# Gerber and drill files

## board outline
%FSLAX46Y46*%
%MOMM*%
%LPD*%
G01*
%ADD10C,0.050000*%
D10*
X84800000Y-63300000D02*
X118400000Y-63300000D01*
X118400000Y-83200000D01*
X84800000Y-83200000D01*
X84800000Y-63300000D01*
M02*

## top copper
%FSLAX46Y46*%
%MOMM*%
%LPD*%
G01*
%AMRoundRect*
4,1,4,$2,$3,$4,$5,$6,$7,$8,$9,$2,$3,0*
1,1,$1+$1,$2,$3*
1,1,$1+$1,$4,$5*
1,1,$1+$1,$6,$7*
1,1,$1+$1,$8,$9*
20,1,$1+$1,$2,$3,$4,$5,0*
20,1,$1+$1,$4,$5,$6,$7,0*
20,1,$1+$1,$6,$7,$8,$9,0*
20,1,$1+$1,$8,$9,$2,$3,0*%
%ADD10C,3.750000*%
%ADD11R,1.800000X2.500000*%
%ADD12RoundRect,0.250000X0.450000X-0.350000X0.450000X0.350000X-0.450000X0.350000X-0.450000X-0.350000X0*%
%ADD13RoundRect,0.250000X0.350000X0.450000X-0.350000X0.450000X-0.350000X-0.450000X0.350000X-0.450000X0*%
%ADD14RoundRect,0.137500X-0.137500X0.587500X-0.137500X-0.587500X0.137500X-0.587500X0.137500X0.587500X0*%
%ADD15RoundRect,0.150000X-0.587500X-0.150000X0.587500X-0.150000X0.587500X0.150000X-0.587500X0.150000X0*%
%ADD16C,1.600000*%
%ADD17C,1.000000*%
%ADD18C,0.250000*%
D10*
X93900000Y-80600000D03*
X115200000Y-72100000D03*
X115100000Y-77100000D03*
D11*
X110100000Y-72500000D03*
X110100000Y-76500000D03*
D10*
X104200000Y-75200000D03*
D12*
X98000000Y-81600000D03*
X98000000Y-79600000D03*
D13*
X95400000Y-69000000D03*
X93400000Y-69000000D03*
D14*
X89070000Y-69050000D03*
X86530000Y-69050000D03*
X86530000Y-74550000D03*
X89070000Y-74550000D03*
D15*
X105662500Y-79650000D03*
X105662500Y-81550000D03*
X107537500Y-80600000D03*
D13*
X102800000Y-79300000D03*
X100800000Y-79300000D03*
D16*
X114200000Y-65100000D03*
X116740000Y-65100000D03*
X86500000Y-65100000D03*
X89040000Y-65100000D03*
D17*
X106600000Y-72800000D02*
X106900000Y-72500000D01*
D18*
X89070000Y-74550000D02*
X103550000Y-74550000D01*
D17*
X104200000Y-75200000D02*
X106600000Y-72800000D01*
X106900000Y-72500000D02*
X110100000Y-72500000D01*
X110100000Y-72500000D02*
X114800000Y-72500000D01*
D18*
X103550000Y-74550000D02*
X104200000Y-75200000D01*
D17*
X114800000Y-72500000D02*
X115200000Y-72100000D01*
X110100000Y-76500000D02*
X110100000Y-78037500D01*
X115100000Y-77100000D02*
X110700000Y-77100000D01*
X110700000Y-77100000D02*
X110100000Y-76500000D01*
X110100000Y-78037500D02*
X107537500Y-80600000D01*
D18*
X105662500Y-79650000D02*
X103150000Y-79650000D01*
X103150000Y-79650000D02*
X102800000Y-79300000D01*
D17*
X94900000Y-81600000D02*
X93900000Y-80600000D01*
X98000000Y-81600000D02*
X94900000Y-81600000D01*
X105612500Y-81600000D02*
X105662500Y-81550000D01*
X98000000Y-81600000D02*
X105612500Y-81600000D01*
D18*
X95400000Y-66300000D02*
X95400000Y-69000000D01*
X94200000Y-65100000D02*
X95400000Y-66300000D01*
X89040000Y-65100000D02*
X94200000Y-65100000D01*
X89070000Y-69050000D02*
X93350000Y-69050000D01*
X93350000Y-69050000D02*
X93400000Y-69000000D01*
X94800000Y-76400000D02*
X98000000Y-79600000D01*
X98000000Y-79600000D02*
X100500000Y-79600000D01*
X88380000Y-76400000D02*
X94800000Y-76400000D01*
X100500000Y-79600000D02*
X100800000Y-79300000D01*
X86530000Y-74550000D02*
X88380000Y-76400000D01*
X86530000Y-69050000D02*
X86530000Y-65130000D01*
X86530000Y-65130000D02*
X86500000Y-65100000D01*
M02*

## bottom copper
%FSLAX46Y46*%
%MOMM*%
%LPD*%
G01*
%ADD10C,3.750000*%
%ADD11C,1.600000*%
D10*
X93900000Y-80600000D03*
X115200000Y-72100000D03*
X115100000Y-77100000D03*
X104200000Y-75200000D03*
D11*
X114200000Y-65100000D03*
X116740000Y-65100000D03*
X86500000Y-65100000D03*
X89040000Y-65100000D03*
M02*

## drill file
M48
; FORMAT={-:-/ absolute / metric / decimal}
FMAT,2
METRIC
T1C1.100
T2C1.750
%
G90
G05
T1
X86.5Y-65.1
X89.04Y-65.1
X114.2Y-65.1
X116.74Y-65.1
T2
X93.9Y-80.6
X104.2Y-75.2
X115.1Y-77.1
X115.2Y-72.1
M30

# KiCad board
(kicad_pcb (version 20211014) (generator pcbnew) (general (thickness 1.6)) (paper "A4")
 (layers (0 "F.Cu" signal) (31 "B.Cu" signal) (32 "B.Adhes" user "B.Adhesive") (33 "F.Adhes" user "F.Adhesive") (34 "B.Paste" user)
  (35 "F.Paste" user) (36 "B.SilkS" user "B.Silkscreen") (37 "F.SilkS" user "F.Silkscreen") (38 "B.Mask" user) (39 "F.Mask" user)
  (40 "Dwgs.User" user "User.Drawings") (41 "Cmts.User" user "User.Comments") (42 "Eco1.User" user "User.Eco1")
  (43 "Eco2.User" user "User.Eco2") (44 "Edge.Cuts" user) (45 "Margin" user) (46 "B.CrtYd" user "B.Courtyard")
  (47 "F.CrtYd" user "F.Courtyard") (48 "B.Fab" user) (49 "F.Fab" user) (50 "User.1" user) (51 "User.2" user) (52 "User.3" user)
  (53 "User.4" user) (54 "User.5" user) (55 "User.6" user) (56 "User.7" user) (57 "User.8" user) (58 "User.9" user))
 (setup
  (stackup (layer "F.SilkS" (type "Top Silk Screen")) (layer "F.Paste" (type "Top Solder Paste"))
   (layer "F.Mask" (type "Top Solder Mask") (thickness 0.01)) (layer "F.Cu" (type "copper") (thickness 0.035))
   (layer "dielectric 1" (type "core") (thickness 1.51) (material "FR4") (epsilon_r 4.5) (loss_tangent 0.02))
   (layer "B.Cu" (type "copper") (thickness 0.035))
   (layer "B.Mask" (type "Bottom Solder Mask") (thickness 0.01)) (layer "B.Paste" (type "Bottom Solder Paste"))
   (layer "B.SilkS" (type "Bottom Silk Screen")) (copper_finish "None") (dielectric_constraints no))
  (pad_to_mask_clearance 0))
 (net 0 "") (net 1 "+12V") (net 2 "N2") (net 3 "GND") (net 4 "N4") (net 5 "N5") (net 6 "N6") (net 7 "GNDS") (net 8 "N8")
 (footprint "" (layer "F.Cu") (at 93.9 80.6)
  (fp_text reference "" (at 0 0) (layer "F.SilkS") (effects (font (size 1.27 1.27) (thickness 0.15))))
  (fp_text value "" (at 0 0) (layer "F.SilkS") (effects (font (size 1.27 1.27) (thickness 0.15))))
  (pad "3" thru_hole circle (at 0 0 270) (size 3.75 3.75) (drill 1.75) (layers *.Cu *.Mask "B.SilkS")))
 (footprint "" (layer "F.Cu") (at 115.2 72.1)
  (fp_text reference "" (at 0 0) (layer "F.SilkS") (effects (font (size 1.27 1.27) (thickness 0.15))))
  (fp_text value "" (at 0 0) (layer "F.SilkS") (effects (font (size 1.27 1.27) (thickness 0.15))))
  (pad "3" thru_hole circle (at 0 0 270) (size 3.75 3.75) (drill 1.75) (layers *.Cu *.Mask "B.SilkS")))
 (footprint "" (layer "F.Cu") (at 115.1 77.1)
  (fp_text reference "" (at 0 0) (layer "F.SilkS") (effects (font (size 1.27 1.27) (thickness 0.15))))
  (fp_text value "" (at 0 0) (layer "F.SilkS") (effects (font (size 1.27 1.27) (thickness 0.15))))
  (pad "3" thru_hole circle (at 0 0 270) (size 3.75 3.75) (drill 1.75) (layers *.Cu *.Mask "B.SilkS")))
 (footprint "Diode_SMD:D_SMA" (layer "F.Cu") (at 110.1 74.5 -90)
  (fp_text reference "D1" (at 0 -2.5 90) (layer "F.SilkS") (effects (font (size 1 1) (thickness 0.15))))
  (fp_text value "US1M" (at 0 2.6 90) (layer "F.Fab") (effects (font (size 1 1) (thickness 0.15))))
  (pad "1" smd rect (at -2 0 270) (size 2.5 1.8) (layers "F.Cu" "F.Paste" "F.Mask") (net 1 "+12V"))
  (pad "2" smd rect (at 2 0 270) (size 2.5 1.8) (layers "F.Cu" "F.Paste" "F.Mask") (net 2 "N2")))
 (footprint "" (layer "F.Cu") (at 104.2 75.2)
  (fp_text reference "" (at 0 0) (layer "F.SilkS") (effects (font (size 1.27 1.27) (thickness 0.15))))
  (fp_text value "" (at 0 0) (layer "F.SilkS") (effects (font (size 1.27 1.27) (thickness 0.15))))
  (pad "3" thru_hole circle (at 0 0 270) (size 3.75 3.75) (drill 1.75) (layers *.Cu *.Mask "B.SilkS")))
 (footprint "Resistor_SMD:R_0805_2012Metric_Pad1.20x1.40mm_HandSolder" (layer "F.Cu") (at 98 80.6 90)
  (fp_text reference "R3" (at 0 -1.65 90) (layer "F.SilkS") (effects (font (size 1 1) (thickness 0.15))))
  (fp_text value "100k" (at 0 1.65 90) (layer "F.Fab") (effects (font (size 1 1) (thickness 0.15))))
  (pad "1" smd roundrect (at -1 0 90) (size 1.2 1.4) (layers "F.Cu" "F.Paste" "F.Mask") (roundrect_rratio 0.2083333333) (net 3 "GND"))
  (pad "2" smd roundrect (at 1 0 90) (size 1.2 1.4) (layers "F.Cu" "F.Paste" "F.Mask") (roundrect_rratio 0.2083333333) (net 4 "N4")))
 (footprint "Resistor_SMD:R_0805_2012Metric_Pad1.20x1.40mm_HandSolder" (layer "F.Cu") (at 94.4 69 180)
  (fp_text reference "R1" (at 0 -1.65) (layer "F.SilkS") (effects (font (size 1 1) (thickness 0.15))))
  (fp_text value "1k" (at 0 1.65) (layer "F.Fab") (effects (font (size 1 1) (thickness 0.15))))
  (pad "1" smd roundrect (at -1 0 180) (size 1.2 1.4) (layers "F.Cu" "F.Paste" "F.Mask") (roundrect_rratio 0.2083333333) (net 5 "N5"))
  (pad "2" smd roundrect (at 1 0 180) (size 1.2 1.4) (layers "F.Cu" "F.Paste" "F.Mask") (roundrect_rratio 0.2083333333) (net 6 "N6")))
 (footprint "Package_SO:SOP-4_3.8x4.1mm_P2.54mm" (layer "F.Cu") (at 87.8 71.8 -90)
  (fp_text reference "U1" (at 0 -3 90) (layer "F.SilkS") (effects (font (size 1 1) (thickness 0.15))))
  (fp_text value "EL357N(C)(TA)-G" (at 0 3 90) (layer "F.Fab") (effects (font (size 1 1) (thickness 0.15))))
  (pad "1" smd roundrect (at -2.75 -1.27 270) (size 1.45 0.55) (layers "F.Cu" "F.Paste" "F.Mask") (roundrect_rratio 0.25) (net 6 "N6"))
  (pad "2" smd roundrect (at -2.75 1.27 270) (size 1.45 0.55) (layers "F.Cu" "F.Paste" "F.Mask") (roundrect_rratio 0.25) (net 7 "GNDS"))
  (pad "3" smd roundrect (at 2.75 1.27 270) (size 1.45 0.55) (layers "F.Cu" "F.Paste" "F.Mask") (roundrect_rratio 0.25) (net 4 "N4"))
  (pad "4" smd roundrect (at 2.75 -1.27 270) (size 1.45 0.55) (layers "F.Cu" "F.Paste" "F.Mask") (roundrect_rratio 0.25) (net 1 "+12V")))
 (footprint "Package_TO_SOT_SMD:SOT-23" (layer "F.Cu") (at 106.6 80.6)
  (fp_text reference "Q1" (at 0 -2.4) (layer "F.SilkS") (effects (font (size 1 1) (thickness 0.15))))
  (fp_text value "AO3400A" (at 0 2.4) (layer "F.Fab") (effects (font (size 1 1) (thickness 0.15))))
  (pad "1" smd roundrect (at -0.9375 -0.95) (size 1.475 0.6) (layers "F.Cu" "F.Paste" "F.Mask") (roundrect_rratio 0.25) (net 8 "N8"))
  (pad "2" smd roundrect (at -0.9375 0.95) (size 1.475 0.6) (layers "F.Cu" "F.Paste" "F.Mask") (roundrect_rratio 0.25) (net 3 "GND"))
  (pad "3" smd roundrect (at 0.9375 0) (size 1.475 0.6) (layers "F.Cu" "F.Paste" "F.Mask") (roundrect_rratio 0.25) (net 2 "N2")))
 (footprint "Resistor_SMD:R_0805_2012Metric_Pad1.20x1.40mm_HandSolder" (layer "F.Cu") (at 101.8 79.3 180)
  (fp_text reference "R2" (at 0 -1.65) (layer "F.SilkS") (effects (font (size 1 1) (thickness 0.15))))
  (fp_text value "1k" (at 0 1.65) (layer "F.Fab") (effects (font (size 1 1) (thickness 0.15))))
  (pad "1" smd roundrect (at -1 0 180) (size 1.2 1.4) (layers "F.Cu" "F.Paste" "F.Mask") (roundrect_rratio 0.2083333333) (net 8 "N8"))
  (pad "2" smd roundrect (at 1 0 180) (size 1.2 1.4) (layers "F.Cu" "F.Paste" "F.Mask") (roundrect_rratio 0.2083333333) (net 4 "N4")))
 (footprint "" (layer "B.Cu") (at 114.2 65.1 180)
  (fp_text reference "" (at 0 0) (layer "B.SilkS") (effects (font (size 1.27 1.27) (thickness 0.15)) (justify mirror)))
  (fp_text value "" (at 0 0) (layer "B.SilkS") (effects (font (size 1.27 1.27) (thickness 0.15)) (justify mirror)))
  (pad "3" thru_hole circle (at 0 0 270) (size 1.6 1.6) (drill 1.1) (layers *.Cu *.Mask "B.SilkS")))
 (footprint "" (layer "B.Cu") (at 116.74 65.1 180)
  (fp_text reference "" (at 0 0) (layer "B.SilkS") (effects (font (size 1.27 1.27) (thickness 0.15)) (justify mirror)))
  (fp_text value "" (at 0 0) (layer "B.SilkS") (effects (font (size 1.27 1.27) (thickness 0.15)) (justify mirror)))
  (pad "12" thru_hole circle (at 0 0 270) (size 1.6 1.6) (drill 1.1) (layers *.Cu *.Mask "B.SilkS")))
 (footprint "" (layer "B.Cu") (at 86.5 65.1 180)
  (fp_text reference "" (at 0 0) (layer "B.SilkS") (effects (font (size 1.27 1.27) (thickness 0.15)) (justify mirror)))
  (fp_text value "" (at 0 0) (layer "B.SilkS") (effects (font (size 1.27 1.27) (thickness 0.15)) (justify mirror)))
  (pad "3" thru_hole circle (at 0 0 270) (size 1.6 1.6) (drill 1.1) (layers *.Cu *.Mask "B.SilkS")))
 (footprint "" (layer "B.Cu") (at 89.04 65.1 180)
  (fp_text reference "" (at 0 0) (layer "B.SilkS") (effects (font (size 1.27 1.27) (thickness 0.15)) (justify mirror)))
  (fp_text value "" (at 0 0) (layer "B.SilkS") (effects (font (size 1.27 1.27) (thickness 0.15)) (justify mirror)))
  (pad "12" thru_hole circle (at 0 0 270) (size 1.6 1.6) (drill 1.1) (layers *.Cu *.Mask "B.SilkS")))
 (gr_rect (start 84.8 63.3) (end 118.4 83.2) (layer "Edge.Cuts") (width 0.05) (fill none))
 (segment (start 106.6 72.8) (end 106.9 72.5) (width 1) (layer "F.Cu") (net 1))
 (segment (start 89.07 74.55) (end 103.55 74.55) (width 0.25) (layer "F.Cu") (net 1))
 (segment (start 104.2 75.2) (end 106.6 72.8) (width 1) (layer "F.Cu") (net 1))
 (segment (start 106.9 72.5) (end 110.1 72.5) (width 1) (layer "F.Cu") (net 1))
 (segment (start 110.1 72.5) (end 114.8 72.5) (width 1) (layer "F.Cu") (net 1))
 (segment (start 103.55 74.55) (end 104.2 75.2) (width 0.25) (layer "F.Cu") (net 1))
 (segment (start 114.8 72.5) (end 115.2 72.1) (width 1) (layer "F.Cu") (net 1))
 (segment (start 110.1 76.5) (end 110.1 78.0375) (width 1) (layer "F.Cu") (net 2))
 (segment (start 115.1 77.1) (end 110.7 77.1) (width 1) (layer "F.Cu") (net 2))
 (segment (start 110.7 77.1) (end 110.1 76.5) (width 1) (layer "F.Cu") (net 2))
 (segment (start 110.1 78.0375) (end 107.5375 80.6) (width 1) (layer "F.Cu") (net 2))
 (segment (start 105.6625 79.65) (end 103.15 79.65) (width 0.25) (layer "F.Cu") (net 8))
 (segment (start 103.15 79.65) (end 102.8 79.3) (width 0.25) (layer "F.Cu") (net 8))
 (segment (start 94.9 81.6) (end 93.9 80.6) (width 1) (layer "F.Cu") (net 3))
 (segment (start 98 81.6) (end 94.9 81.6) (width 1) (layer "F.Cu") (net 3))
 (segment (start 105.6125 81.6) (end 105.6625 81.55) (width 1) (layer "F.Cu") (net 3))
 (segment (start 98 81.6) (end 105.6125 81.6) (width 1) (layer "F.Cu") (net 3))
 (segment (start 95.4 66.3) (end 95.4 69) (width 0.25) (layer "F.Cu") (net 5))
 (segment (start 94.2 65.1) (end 95.4 66.3) (width 0.25) (layer "F.Cu") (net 5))
 (segment (start 89.04 65.1) (end 94.2 65.1) (width 0.25) (layer "F.Cu") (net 5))
 (segment (start 89.07 69.05) (end 93.35 69.05) (width 0.25) (layer "F.Cu") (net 6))
 (segment (start 93.35 69.05) (end 93.4 69) (width 0.25) (layer "F.Cu") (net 6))
 (segment (start 94.8 76.4) (end 98 79.6) (width 0.25) (layer "F.Cu") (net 4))
 (segment (start 98 79.6) (end 100.5 79.6) (width 0.25) (layer "F.Cu") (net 4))
 (segment (start 88.38 76.4) (end 94.8 76.4) (width 0.25) (layer "F.Cu") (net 4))
 (segment (start 100.5 79.6) (end 100.8 79.3) (width 0.25) (layer "F.Cu") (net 4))
 (segment (start 86.53 74.55) (end 88.38 76.4) (width 0.25) (layer "F.Cu") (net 4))
 (segment (start 86.53 69.05) (end 86.53 65.13) (width 0.25) (layer "F.Cu") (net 7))
 (segment (start 86.53 65.13) (end 86.5 65.1) (width 0.25) (layer "F.Cu") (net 7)))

